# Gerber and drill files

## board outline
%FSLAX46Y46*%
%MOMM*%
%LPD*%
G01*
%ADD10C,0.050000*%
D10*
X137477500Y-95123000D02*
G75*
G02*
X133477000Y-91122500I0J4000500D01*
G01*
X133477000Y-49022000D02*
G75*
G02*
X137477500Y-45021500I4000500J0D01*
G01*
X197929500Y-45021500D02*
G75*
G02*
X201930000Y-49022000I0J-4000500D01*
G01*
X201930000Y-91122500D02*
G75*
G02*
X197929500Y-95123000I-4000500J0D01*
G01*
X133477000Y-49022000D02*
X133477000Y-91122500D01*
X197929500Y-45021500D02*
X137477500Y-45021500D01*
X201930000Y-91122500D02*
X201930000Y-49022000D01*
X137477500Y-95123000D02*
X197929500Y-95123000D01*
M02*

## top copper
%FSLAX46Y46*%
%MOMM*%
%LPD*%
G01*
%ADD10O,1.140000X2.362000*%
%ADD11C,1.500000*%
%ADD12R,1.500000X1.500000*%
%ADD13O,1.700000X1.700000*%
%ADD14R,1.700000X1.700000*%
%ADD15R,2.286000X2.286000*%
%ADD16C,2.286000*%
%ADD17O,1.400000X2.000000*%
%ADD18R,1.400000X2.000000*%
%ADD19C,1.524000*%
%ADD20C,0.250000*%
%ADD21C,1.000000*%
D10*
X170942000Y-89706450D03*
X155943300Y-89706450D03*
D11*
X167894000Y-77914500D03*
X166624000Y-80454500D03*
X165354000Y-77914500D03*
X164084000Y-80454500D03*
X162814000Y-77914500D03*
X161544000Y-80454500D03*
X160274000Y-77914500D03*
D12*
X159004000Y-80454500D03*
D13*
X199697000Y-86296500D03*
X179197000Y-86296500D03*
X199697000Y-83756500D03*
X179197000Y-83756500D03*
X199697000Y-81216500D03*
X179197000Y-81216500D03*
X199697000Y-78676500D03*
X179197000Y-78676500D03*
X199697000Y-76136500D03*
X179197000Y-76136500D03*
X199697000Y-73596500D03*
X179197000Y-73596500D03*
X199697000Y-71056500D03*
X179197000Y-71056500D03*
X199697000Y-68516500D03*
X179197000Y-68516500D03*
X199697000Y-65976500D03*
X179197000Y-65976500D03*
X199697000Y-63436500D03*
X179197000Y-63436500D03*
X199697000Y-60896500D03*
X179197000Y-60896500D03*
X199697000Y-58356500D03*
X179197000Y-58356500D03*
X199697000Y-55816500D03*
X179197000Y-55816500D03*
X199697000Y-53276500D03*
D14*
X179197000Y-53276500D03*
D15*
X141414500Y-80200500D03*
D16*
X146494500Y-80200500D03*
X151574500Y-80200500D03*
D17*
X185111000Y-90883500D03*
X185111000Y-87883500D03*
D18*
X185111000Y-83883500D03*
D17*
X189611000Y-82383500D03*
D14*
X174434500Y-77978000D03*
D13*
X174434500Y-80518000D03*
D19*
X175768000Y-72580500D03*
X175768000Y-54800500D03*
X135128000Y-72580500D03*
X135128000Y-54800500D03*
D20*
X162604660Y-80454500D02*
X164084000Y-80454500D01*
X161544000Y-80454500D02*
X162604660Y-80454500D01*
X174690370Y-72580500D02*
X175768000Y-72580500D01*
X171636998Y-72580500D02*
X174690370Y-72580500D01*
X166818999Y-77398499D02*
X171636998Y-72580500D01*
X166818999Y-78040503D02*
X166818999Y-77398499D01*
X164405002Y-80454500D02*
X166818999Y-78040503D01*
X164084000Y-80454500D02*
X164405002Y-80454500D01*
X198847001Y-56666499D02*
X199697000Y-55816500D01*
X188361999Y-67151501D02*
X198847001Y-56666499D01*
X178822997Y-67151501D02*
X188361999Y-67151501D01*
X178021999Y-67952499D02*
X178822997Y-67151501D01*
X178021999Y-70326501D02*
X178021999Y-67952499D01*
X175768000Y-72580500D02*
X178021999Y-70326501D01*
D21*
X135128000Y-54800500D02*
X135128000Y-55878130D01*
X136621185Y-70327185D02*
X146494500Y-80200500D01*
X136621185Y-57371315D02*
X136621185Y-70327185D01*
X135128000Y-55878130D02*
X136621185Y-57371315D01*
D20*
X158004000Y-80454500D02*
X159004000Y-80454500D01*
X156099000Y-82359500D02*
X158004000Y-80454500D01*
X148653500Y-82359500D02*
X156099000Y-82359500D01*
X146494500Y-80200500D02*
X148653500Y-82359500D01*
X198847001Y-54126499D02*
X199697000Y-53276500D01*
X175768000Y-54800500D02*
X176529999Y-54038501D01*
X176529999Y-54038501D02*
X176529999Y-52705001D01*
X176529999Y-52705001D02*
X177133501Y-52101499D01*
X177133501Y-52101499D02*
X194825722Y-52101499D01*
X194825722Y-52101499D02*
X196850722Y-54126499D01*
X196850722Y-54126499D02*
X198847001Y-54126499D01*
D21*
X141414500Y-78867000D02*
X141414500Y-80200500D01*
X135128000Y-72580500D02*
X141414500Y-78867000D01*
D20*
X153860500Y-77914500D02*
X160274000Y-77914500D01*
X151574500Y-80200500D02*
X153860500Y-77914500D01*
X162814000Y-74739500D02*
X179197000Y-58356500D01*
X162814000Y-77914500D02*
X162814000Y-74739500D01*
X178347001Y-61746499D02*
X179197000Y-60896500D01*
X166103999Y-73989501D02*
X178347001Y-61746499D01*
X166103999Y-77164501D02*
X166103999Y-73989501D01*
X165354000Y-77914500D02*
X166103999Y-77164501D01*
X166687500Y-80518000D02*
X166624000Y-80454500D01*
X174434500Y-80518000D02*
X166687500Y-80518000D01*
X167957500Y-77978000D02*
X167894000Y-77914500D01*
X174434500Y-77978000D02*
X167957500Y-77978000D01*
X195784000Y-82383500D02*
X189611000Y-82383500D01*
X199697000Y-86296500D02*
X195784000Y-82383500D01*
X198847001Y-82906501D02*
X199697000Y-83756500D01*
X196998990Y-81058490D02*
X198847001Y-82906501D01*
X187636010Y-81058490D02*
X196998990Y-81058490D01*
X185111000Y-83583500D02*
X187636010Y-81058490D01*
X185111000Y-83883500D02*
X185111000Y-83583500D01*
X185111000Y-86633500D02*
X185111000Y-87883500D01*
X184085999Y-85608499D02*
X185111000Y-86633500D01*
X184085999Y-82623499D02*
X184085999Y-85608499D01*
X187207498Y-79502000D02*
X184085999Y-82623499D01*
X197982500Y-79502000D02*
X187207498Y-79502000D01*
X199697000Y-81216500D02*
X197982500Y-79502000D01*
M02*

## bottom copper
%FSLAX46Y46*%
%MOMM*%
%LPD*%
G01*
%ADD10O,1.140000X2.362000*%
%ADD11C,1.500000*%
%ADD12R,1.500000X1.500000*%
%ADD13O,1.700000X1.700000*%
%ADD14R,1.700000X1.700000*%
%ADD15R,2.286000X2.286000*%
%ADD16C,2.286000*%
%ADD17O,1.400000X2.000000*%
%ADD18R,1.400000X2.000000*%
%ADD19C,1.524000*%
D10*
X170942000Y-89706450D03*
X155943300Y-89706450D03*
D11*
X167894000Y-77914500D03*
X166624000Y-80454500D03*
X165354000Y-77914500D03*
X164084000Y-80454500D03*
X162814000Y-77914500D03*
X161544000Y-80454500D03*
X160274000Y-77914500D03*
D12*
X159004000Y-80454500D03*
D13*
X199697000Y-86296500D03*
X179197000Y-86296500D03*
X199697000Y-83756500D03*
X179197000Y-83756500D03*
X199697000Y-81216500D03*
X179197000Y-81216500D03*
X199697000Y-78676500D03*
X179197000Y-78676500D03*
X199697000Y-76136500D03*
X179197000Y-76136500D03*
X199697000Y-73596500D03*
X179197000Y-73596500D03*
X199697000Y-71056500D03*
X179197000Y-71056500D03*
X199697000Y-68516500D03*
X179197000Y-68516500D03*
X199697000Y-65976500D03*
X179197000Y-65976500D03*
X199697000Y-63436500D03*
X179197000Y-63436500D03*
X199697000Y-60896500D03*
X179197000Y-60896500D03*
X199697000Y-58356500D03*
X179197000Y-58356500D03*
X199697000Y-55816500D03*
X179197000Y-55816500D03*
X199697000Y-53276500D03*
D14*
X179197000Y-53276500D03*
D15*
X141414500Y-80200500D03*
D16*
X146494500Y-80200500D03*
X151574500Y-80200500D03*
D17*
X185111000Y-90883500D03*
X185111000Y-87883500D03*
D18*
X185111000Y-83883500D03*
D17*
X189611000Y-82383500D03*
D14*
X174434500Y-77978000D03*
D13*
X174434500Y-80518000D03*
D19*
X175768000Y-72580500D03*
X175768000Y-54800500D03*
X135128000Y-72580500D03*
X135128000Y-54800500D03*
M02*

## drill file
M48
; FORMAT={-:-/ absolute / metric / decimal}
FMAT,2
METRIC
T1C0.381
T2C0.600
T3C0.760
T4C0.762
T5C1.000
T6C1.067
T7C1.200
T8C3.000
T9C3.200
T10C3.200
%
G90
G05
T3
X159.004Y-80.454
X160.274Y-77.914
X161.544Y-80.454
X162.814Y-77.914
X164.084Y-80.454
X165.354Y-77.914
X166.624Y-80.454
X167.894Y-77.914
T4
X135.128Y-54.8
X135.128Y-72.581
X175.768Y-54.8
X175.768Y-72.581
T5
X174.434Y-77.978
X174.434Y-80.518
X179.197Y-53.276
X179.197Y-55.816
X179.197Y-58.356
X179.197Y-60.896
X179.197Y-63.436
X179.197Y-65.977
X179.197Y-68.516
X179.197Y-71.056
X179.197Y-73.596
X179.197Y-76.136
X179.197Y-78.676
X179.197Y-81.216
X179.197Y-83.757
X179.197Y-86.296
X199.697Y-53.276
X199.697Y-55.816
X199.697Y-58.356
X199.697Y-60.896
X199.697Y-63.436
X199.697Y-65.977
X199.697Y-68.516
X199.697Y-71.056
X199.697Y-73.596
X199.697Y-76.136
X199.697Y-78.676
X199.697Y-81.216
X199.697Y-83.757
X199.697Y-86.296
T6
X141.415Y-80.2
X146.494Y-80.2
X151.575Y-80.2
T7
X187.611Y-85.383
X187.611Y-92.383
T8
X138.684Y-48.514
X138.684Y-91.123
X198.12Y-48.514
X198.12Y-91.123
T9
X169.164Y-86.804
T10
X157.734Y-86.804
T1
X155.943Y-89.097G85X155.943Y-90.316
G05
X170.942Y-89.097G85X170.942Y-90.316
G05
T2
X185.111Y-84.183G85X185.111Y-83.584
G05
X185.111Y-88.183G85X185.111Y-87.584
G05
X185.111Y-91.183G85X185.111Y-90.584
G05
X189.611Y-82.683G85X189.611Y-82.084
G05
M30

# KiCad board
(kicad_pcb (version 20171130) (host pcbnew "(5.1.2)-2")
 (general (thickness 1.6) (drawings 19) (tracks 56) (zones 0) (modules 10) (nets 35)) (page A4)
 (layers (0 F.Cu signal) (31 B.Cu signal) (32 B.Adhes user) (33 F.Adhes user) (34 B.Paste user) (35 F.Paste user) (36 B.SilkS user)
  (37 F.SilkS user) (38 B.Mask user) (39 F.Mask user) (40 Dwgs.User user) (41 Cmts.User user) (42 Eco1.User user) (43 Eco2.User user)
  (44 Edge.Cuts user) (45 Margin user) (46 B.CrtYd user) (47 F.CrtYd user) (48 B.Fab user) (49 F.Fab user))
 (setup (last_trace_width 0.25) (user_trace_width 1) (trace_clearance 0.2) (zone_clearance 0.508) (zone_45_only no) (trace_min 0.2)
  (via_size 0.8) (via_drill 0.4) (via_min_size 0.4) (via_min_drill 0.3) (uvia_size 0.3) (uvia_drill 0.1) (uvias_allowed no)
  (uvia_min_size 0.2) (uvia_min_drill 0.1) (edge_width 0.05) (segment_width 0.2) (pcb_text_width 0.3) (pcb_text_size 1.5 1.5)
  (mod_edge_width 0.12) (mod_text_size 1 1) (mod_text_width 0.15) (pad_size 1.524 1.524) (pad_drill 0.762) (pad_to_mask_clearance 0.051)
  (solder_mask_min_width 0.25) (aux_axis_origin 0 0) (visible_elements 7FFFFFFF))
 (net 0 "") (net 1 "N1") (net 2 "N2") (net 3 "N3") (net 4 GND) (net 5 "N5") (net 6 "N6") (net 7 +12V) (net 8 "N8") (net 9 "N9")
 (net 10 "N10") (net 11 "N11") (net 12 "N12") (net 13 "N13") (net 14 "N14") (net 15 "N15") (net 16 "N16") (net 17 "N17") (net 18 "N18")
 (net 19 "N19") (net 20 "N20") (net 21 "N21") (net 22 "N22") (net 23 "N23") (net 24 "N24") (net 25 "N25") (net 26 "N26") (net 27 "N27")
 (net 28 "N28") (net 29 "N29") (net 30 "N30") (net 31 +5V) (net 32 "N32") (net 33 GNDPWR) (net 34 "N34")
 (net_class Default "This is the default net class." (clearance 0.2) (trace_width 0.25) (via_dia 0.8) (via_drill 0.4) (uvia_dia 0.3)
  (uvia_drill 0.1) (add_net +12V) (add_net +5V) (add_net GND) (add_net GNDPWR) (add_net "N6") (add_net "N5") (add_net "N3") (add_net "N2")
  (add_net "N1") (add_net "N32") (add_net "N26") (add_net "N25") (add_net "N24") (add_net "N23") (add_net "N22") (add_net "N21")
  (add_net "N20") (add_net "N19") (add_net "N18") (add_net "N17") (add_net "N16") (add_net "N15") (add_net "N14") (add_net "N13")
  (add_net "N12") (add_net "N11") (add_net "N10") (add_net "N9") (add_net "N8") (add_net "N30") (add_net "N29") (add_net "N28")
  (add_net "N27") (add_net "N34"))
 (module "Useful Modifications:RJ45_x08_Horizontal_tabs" (layer F.Cu) (at 159.004 80.4545)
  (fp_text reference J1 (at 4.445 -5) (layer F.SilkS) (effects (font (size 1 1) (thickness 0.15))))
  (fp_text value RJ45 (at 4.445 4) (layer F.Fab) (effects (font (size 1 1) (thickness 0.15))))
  (pad 10 thru_hole oval (at 11.938 9.25195) (size 1.14 2.362) (drill oval 0.381 1.6) (layers *.Cu *.Mask))
  (pad 9 thru_hole oval (at -3.0607 9.25195) (size 1.14 2.362) (drill oval 0.381 1.6) (layers *.Cu *.Mask))
  (pad 8 thru_hole circle (at 8.89 -2.54) (size 1.5 1.5) (drill 0.76) (layers *.Cu *.Mask) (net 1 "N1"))
  (pad 7 thru_hole circle (at 7.62 0) (size 1.5 1.5) (drill 0.76) (layers *.Cu *.Mask) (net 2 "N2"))
  (pad 6 thru_hole circle (at 6.35 -2.54) (size 1.5 1.5) (drill 0.76) (layers *.Cu *.Mask) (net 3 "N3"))
  (pad 5 thru_hole circle (at 5.08 0) (size 1.5 1.5) (drill 0.76) (layers *.Cu *.Mask) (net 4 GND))
  (pad 4 thru_hole circle (at 3.81 -2.54) (size 1.5 1.5) (drill 0.76) (layers *.Cu *.Mask) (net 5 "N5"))
  (pad 3 thru_hole circle (at 2.54 0) (size 1.5 1.5) (drill 0.76) (layers *.Cu *.Mask) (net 4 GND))
  (pad 2 thru_hole circle (at 1.27 -2.54) (size 1.5 1.5) (drill 0.76) (layers *.Cu *.Mask) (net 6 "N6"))
  (pad 1 thru_hole rect (at 0 0) (size 1.5 1.5) (drill 0.76) (layers *.Cu *.Mask) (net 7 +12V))
  (pad "" np_thru_hole circle (at -1.27 6.35) (size 3.200001 3.200001) (drill 3.200001) (layers *.Cu *.Mask))
  (pad "" np_thru_hole circle (at 10.16 6.35) (size 3.2 3.2) (drill 3.2) (layers *.Cu *.Mask)))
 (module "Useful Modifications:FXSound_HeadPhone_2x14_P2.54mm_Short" (layer F.Cu) (at 179.197 53.2765)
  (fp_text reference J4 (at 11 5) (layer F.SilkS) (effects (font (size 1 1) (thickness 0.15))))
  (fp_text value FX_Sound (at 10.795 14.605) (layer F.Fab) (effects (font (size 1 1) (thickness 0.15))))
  (pad 28 thru_hole oval (at 20.5 33.02) (size 1.7 1.7) (drill 1) (layers *.Cu *.Mask) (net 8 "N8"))
  (pad 27 thru_hole oval (at 0 33.02) (size 1.7 1.7) (drill 1) (layers *.Cu *.Mask) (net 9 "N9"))
  (pad 26 thru_hole oval (at 20.5 30.48) (size 1.7 1.7) (drill 1) (layers *.Cu *.Mask) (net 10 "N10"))
  (pad 25 thru_hole oval (at 0 30.48) (size 1.7 1.7) (drill 1) (layers *.Cu *.Mask) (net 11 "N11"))
  (pad 24 thru_hole oval (at 20.5 27.94) (size 1.7 1.7) (drill 1) (layers *.Cu *.Mask) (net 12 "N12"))
  (pad 23 thru_hole oval (at 0 27.94) (size 1.7 1.7) (drill 1) (layers *.Cu *.Mask) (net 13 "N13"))
  (pad 22 thru_hole oval (at 20.5 25.4) (size 1.7 1.7) (drill 1) (layers *.Cu *.Mask) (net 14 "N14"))
  (pad 21 thru_hole oval (at 0 25.4) (size 1.7 1.7) (drill 1) (layers *.Cu *.Mask) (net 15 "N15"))
  (pad 20 thru_hole oval (at 20.5 22.86) (size 1.7 1.7) (drill 1) (layers *.Cu *.Mask) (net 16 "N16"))
  (pad 19 thru_hole oval (at 0 22.86) (size 1.7 1.7) (drill 1) (layers *.Cu *.Mask) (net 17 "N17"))
  (pad 18 thru_hole oval (at 20.5 20.32) (size 1.7 1.7) (drill 1) (layers *.Cu *.Mask) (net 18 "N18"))
  (pad 17 thru_hole oval (at 0 20.32) (size 1.7 1.7) (drill 1) (layers *.Cu *.Mask) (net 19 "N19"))
  (pad 16 thru_hole oval (at 20.5 17.78) (size 1.7 1.7) (drill 1) (layers *.Cu *.Mask) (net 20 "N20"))
  (pad 15 thru_hole oval (at 0 17.78) (size 1.7 1.7) (drill 1) (layers *.Cu *.Mask) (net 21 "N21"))
  (pad 14 thru_hole oval (at 20.5 15.24) (size 1.7 1.7) (drill 1) (layers *.Cu *.Mask) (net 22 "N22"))
  (pad 13 thru_hole oval (at 0 15.24) (size 1.7 1.7) (drill 1) (layers *.Cu *.Mask) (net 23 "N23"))
  (pad 12 thru_hole oval (at 20.5 12.7) (size 1.7 1.7) (drill 1) (layers *.Cu *.Mask) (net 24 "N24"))
  (pad 11 thru_hole oval (at 0 12.7) (size 1.7 1.7) (drill 1) (layers *.Cu *.Mask) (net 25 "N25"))
  (pad 10 thru_hole oval (at 20.5 10.16) (size 1.7 1.7) (drill 1) (layers *.Cu *.Mask) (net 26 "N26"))
  (pad 9 thru_hole oval (at 0 10.16) (size 1.7 1.7) (drill 1) (layers *.Cu *.Mask) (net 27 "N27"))
  (pad 8 thru_hole oval (at 20.5 7.62) (size 1.7 1.7) (drill 1) (layers *.Cu *.Mask) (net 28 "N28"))
  (pad 7 thru_hole oval (at 0 7.62) (size 1.7 1.7) (drill 1) (layers *.Cu *.Mask) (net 3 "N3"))
  (pad 6 thru_hole oval (at 20.5 5.08) (size 1.7 1.7) (drill 1) (layers *.Cu *.Mask) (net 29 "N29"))
  (pad 5 thru_hole oval (at 0 5.08) (size 1.7 1.7) (drill 1) (layers *.Cu *.Mask) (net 5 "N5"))
  (pad 4 thru_hole oval (at 20.5 2.54) (size 1.7 1.7) (drill 1) (layers *.Cu *.Mask) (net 4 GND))
  (pad 3 thru_hole oval (at 0 2.54) (size 1.7 1.7) (drill 1) (layers *.Cu *.Mask) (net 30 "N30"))
  (pad 2 thru_hole oval (at 20.5 0) (size 1.7 1.7) (drill 1) (layers *.Cu *.Mask) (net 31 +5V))
  (pad 1 thru_hole rect (at 0 0) (size 1.7 1.7) (drill 1) (layers *.Cu *.Mask) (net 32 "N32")))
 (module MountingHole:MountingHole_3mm (layer F.Cu) (at 138.684 48.514)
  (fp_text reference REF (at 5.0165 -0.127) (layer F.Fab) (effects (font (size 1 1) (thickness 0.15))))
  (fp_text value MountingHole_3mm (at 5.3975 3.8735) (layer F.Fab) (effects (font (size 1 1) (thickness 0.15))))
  (pad 1 np_thru_hole circle (at 0 0) (size 3 3) (drill 3) (layers *.Cu *.Mask)))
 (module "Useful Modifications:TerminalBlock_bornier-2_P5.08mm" (layer F.Cu) (at 141.4145 80.2005)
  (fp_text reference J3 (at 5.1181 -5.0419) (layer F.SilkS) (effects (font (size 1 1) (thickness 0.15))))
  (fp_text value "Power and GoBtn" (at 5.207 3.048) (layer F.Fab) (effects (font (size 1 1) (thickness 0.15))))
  (pad 1 thru_hole rect (at 0 0) (size 2.286 2.286) (drill 1.0668) (layers *.Cu *.Mask) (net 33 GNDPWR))
  (pad 2 thru_hole circle (at 5.08 0) (size 2.286 2.286) (drill 1.0668) (layers *.Cu *.Mask) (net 7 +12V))
  (pad 3 thru_hole circle (at 10.16 0) (size 2.286 2.286) (drill 1.0668) (layers *.Cu *.Mask) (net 6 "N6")))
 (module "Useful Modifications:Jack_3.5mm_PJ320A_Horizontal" (layer F.Cu) (at 189.611 83.8835 180)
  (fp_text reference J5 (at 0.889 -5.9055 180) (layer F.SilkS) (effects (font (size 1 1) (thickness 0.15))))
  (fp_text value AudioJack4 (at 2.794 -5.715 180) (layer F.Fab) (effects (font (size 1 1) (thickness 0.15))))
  (pad "" np_thru_hole circle (at 2 -1.5 90) (size 1.2 1.2) (drill 1.2) (layers *.Cu *.Mask))
  (pad "" np_thru_hole circle (at 2 -8.5 90) (size 1.2 1.2) (drill 1.2) (layers *.Cu *.Mask))
  (pad R2 thru_hole oval (at 4.5 -7 90) (size 2 1.4) (drill oval 1.2 0.6) (layers *.Cu *.Mask) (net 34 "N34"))
  (pad R1 thru_hole oval (at 4.5 -4 90) (size 2 1.4) (drill oval 1.2 0.6) (layers *.Cu *.Mask) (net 12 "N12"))
  (pad T thru_hole rect (at 4.5 0 90) (size 2 1.4) (drill oval 1.2 0.6) (layers *.Cu *.Mask) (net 10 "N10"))
  (pad S thru_hole oval (at 0 1.5 90) (size 2 1.4) (drill oval 1.2 0.6) (layers *.Cu *.Mask) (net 8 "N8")))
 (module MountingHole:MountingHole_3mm (layer F.Cu) (at 198.12 48.514)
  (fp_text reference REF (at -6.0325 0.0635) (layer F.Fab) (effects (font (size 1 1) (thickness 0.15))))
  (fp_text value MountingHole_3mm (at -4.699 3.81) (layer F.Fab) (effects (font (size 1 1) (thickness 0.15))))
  (pad 1 np_thru_hole circle (at 0 0) (size 3 3) (drill 3) (layers *.Cu *.Mask)))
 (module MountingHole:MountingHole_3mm (layer F.Cu) (at 198.12 91.1225)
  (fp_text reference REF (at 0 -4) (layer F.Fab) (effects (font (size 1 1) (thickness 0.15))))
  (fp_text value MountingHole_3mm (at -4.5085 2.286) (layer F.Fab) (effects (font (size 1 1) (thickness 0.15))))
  (pad 1 np_thru_hole circle (at 0 0) (size 3 3) (drill 3) (layers *.Cu *.Mask)))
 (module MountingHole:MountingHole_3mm (layer F.Cu) (at 138.684 91.1225)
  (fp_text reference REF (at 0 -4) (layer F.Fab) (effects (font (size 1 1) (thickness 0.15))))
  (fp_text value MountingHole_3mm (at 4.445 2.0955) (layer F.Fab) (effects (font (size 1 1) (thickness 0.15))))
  (pad 1 np_thru_hole circle (at 0 0) (size 3 3) (drill 3) (layers *.Cu *.Mask)))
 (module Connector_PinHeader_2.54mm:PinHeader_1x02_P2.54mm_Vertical (layer F.Cu) (at 174.4345 77.978)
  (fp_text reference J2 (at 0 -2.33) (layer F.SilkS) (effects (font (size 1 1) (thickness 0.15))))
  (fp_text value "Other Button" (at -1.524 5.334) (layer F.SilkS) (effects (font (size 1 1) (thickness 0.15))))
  (pad 1 thru_hole rect (at 0 0) (size 1.7 1.7) (drill 1) (layers *.Cu *.Mask) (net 1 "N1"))
  (pad 2 thru_hole oval (at 0 2.54) (size 1.7 1.7) (drill 1) (layers *.Cu *.Mask) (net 2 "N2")))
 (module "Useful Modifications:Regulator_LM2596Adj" (layer F.Cu) (at 157.988 64.9605)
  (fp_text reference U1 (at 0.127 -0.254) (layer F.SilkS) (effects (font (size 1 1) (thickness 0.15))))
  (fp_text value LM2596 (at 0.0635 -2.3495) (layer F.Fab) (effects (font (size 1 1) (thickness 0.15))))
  (pad 6 thru_hole circle (at 17.78 7.62) (size 1.524 1.524) (drill 0.762) (layers *.Cu *.Mask) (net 4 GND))
  (pad 4 thru_hole circle (at 17.78 -10.16) (size 1.524 1.524) (drill 0.762) (layers *.Cu *.Mask) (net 31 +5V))
  (pad 1 thru_hole circle (at -22.86 7.62) (size 1.524 1.524) (drill 0.762) (layers *.Cu *.Mask) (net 33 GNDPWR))
  (pad 2 thru_hole circle (at -22.86 -10.16) (size 1.524 1.524) (drill 0.762) (layers *.Cu *.Mask) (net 7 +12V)))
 (gr_arc (start 137.4775 91.1225) (end 133.477 91.1225) (angle -90) (layer Edge.Cuts) (width 0.05))
 (gr_arc (start 137.4775 49.022) (end 137.4775 45.0215) (angle -90) (layer Edge.Cuts) (width 0.05))
 (gr_arc (start 197.9295 49.022) (end 201.93 49.022) (angle -90) (layer Edge.Cuts) (width 0.05))
 (gr_arc (start 197.9295 91.1225) (end 197.9295 95.123) (angle -90) (layer Edge.Cuts) (width 0.05))
 (gr_line (start 133.477 49.022) (end 133.477 91.1225) (layer Edge.Cuts) (width 0.05))
 (gr_line (start 197.9295 45.0215) (end 137.4775 45.0215) (layer Edge.Cuts) (width 0.05))
 (gr_line (start 201.93 91.1225) (end 201.93 49.022) (layer Edge.Cuts) (width 0.05))
 (gr_line (start 137.4775 95.123) (end 197.9295 95.123) (layer Edge.Cuts) (width 0.05))
 (segment (start 162.60466 80.4545) (end 164.084 80.4545) (width 0.25) (layer F.Cu) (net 4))
 (segment (start 161.544 80.4545) (end 162.60466 80.4545) (width 0.25) (layer F.Cu) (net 4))
 (segment (start 174.69037 72.5805) (end 175.768 72.5805) (width 0.25) (layer F.Cu) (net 4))
 (segment (start 171.636998 72.5805) (end 174.69037 72.5805) (width 0.25) (layer F.Cu) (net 4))
 (segment (start 166.818999 77.398499) (end 171.636998 72.5805) (width 0.25) (layer F.Cu) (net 4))
 (segment (start 166.818999 78.040503) (end 166.818999 77.398499) (width 0.25) (layer F.Cu) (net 4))
 (segment (start 164.405002 80.4545) (end 166.818999 78.040503) (width 0.25) (layer F.Cu) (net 4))
 (segment (start 164.084 80.4545) (end 164.405002 80.4545) (width 0.25) (layer F.Cu) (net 4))
 (segment (start 198.847001 56.666499) (end 199.697 55.8165) (width 0.25) (layer F.Cu) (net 4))
 (segment (start 188.361999 67.151501) (end 198.847001 56.666499) (width 0.25) (layer F.Cu) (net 4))
 (segment (start 178.822997 67.151501) (end 188.361999 67.151501) (width 0.25) (layer F.Cu) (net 4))
 (segment (start 178.021999 67.952499) (end 178.822997 67.151501) (width 0.25) (layer F.Cu) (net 4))
 (segment (start 178.021999 70.326501) (end 178.021999 67.952499) (width 0.25) (layer F.Cu) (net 4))
 (segment (start 175.768 72.5805) (end 178.021999 70.326501) (width 0.25) (layer F.Cu) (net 4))
 (segment (start 135.128 54.8005) (end 135.128 55.87813) (width 1) (layer F.Cu) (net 7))
 (segment (start 136.621185 70.327185) (end 146.4945 80.2005) (width 1) (layer F.Cu) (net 7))
 (segment (start 136.621185 57.371315) (end 136.621185 70.327185) (width 1) (layer F.Cu) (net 7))
 (segment (start 135.128 55.87813) (end 136.621185 57.371315) (width 1) (layer F.Cu) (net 7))
 (segment (start 158.004 80.4545) (end 159.004 80.4545) (width 0.25) (layer F.Cu) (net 7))
 (segment (start 156.099 82.3595) (end 158.004 80.4545) (width 0.25) (layer F.Cu) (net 7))
 (segment (start 148.6535 82.3595) (end 156.099 82.3595) (width 0.25) (layer F.Cu) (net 7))
 (segment (start 146.4945 80.2005) (end 148.6535 82.3595) (width 0.25) (layer F.Cu) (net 7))
 (segment (start 198.847001 54.126499) (end 199.697 53.2765) (width 0.25) (layer F.Cu) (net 31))
 (segment (start 175.768 54.8005) (end 176.529999 54.038501) (width 0.25) (layer F.Cu) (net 31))
 (segment (start 176.529999 54.038501) (end 176.529999 52.705001) (width 0.25) (layer F.Cu) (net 31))
 (segment (start 176.529999 52.705001) (end 177.133501 52.101499) (width 0.25) (layer F.Cu) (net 31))
 (segment (start 177.133501 52.101499) (end 194.825722 52.101499) (width 0.25) (layer F.Cu) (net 31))
 (segment (start 194.825722 52.101499) (end 196.850722 54.126499) (width 0.25) (layer F.Cu) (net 31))
 (segment (start 196.850722 54.126499) (end 198.847001 54.126499) (width 0.25) (layer F.Cu) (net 31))
 (segment (start 141.4145 78.867) (end 141.4145 80.2005) (width 1) (layer F.Cu) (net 33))
 (segment (start 135.128 72.5805) (end 141.4145 78.867) (width 1) (layer F.Cu) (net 33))
 (segment (start 153.8605 77.9145) (end 160.274 77.9145) (width 0.25) (layer F.Cu) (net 6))
 (segment (start 151.5745 80.2005) (end 153.8605 77.9145) (width 0.25) (layer F.Cu) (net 6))
 (segment (start 162.814 74.7395) (end 179.197 58.3565) (width 0.25) (layer F.Cu) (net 5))
 (segment (start 162.814 77.9145) (end 162.814 74.7395) (width 0.25) (layer F.Cu) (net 5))
 (segment (start 178.347001 61.746499) (end 179.197 60.8965) (width 0.25) (layer F.Cu) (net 3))
 (segment (start 166.103999 73.989501) (end 178.347001 61.746499) (width 0.25) (layer F.Cu) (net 3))
 (segment (start 166.103999 77.164501) (end 166.103999 73.989501) (width 0.25) (layer F.Cu) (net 3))
 (segment (start 165.354 77.9145) (end 166.103999 77.164501) (width 0.25) (layer F.Cu) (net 3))
 (segment (start 166.6875 80.518) (end 166.624 80.4545) (width 0.25) (layer F.Cu) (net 2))
 (segment (start 174.4345 80.518) (end 166.6875 80.518) (width 0.25) (layer F.Cu) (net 2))
 (segment (start 167.9575 77.978) (end 167.894 77.9145) (width 0.25) (layer F.Cu) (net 1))
 (segment (start 174.4345 77.978) (end 167.9575 77.978) (width 0.25) (layer F.Cu) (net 1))
 (segment (start 195.784 82.3835) (end 189.611 82.3835) (width 0.25) (layer F.Cu) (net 8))
 (segment (start 199.697 86.2965) (end 195.784 82.3835) (width 0.25) (layer F.Cu) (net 8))
 (segment (start 198.847001 82.906501) (end 199.697 83.7565) (width 0.25) (layer F.Cu) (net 10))
 (segment (start 196.99899 81.05849) (end 198.847001 82.906501) (width 0.25) (layer F.Cu) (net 10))
 (segment (start 187.63601 81.05849) (end 196.99899 81.05849) (width 0.25) (layer F.Cu) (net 10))
 (segment (start 185.111 83.5835) (end 187.63601 81.05849) (width 0.25) (layer F.Cu) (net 10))
 (segment (start 185.111 83.8835) (end 185.111 83.5835) (width 0.25) (layer F.Cu) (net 10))
 (segment (start 185.111 86.6335) (end 185.111 87.8835) (width 0.25) (layer F.Cu) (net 12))
 (segment (start 184.085999 85.608499) (end 185.111 86.6335) (width 0.25) (layer F.Cu) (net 12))
 (segment (start 184.085999 82.623499) (end 184.085999 85.608499) (width 0.25) (layer F.Cu) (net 12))
 (segment (start 187.207498 79.502) (end 184.085999 82.623499) (width 0.25) (layer F.Cu) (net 12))
 (segment (start 197.9825 79.502) (end 187.207498 79.502) (width 0.25) (layer F.Cu) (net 12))
 (segment (start 199.697 81.2165) (end 197.9825 79.502) (width 0.25) (layer F.Cu) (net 12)))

